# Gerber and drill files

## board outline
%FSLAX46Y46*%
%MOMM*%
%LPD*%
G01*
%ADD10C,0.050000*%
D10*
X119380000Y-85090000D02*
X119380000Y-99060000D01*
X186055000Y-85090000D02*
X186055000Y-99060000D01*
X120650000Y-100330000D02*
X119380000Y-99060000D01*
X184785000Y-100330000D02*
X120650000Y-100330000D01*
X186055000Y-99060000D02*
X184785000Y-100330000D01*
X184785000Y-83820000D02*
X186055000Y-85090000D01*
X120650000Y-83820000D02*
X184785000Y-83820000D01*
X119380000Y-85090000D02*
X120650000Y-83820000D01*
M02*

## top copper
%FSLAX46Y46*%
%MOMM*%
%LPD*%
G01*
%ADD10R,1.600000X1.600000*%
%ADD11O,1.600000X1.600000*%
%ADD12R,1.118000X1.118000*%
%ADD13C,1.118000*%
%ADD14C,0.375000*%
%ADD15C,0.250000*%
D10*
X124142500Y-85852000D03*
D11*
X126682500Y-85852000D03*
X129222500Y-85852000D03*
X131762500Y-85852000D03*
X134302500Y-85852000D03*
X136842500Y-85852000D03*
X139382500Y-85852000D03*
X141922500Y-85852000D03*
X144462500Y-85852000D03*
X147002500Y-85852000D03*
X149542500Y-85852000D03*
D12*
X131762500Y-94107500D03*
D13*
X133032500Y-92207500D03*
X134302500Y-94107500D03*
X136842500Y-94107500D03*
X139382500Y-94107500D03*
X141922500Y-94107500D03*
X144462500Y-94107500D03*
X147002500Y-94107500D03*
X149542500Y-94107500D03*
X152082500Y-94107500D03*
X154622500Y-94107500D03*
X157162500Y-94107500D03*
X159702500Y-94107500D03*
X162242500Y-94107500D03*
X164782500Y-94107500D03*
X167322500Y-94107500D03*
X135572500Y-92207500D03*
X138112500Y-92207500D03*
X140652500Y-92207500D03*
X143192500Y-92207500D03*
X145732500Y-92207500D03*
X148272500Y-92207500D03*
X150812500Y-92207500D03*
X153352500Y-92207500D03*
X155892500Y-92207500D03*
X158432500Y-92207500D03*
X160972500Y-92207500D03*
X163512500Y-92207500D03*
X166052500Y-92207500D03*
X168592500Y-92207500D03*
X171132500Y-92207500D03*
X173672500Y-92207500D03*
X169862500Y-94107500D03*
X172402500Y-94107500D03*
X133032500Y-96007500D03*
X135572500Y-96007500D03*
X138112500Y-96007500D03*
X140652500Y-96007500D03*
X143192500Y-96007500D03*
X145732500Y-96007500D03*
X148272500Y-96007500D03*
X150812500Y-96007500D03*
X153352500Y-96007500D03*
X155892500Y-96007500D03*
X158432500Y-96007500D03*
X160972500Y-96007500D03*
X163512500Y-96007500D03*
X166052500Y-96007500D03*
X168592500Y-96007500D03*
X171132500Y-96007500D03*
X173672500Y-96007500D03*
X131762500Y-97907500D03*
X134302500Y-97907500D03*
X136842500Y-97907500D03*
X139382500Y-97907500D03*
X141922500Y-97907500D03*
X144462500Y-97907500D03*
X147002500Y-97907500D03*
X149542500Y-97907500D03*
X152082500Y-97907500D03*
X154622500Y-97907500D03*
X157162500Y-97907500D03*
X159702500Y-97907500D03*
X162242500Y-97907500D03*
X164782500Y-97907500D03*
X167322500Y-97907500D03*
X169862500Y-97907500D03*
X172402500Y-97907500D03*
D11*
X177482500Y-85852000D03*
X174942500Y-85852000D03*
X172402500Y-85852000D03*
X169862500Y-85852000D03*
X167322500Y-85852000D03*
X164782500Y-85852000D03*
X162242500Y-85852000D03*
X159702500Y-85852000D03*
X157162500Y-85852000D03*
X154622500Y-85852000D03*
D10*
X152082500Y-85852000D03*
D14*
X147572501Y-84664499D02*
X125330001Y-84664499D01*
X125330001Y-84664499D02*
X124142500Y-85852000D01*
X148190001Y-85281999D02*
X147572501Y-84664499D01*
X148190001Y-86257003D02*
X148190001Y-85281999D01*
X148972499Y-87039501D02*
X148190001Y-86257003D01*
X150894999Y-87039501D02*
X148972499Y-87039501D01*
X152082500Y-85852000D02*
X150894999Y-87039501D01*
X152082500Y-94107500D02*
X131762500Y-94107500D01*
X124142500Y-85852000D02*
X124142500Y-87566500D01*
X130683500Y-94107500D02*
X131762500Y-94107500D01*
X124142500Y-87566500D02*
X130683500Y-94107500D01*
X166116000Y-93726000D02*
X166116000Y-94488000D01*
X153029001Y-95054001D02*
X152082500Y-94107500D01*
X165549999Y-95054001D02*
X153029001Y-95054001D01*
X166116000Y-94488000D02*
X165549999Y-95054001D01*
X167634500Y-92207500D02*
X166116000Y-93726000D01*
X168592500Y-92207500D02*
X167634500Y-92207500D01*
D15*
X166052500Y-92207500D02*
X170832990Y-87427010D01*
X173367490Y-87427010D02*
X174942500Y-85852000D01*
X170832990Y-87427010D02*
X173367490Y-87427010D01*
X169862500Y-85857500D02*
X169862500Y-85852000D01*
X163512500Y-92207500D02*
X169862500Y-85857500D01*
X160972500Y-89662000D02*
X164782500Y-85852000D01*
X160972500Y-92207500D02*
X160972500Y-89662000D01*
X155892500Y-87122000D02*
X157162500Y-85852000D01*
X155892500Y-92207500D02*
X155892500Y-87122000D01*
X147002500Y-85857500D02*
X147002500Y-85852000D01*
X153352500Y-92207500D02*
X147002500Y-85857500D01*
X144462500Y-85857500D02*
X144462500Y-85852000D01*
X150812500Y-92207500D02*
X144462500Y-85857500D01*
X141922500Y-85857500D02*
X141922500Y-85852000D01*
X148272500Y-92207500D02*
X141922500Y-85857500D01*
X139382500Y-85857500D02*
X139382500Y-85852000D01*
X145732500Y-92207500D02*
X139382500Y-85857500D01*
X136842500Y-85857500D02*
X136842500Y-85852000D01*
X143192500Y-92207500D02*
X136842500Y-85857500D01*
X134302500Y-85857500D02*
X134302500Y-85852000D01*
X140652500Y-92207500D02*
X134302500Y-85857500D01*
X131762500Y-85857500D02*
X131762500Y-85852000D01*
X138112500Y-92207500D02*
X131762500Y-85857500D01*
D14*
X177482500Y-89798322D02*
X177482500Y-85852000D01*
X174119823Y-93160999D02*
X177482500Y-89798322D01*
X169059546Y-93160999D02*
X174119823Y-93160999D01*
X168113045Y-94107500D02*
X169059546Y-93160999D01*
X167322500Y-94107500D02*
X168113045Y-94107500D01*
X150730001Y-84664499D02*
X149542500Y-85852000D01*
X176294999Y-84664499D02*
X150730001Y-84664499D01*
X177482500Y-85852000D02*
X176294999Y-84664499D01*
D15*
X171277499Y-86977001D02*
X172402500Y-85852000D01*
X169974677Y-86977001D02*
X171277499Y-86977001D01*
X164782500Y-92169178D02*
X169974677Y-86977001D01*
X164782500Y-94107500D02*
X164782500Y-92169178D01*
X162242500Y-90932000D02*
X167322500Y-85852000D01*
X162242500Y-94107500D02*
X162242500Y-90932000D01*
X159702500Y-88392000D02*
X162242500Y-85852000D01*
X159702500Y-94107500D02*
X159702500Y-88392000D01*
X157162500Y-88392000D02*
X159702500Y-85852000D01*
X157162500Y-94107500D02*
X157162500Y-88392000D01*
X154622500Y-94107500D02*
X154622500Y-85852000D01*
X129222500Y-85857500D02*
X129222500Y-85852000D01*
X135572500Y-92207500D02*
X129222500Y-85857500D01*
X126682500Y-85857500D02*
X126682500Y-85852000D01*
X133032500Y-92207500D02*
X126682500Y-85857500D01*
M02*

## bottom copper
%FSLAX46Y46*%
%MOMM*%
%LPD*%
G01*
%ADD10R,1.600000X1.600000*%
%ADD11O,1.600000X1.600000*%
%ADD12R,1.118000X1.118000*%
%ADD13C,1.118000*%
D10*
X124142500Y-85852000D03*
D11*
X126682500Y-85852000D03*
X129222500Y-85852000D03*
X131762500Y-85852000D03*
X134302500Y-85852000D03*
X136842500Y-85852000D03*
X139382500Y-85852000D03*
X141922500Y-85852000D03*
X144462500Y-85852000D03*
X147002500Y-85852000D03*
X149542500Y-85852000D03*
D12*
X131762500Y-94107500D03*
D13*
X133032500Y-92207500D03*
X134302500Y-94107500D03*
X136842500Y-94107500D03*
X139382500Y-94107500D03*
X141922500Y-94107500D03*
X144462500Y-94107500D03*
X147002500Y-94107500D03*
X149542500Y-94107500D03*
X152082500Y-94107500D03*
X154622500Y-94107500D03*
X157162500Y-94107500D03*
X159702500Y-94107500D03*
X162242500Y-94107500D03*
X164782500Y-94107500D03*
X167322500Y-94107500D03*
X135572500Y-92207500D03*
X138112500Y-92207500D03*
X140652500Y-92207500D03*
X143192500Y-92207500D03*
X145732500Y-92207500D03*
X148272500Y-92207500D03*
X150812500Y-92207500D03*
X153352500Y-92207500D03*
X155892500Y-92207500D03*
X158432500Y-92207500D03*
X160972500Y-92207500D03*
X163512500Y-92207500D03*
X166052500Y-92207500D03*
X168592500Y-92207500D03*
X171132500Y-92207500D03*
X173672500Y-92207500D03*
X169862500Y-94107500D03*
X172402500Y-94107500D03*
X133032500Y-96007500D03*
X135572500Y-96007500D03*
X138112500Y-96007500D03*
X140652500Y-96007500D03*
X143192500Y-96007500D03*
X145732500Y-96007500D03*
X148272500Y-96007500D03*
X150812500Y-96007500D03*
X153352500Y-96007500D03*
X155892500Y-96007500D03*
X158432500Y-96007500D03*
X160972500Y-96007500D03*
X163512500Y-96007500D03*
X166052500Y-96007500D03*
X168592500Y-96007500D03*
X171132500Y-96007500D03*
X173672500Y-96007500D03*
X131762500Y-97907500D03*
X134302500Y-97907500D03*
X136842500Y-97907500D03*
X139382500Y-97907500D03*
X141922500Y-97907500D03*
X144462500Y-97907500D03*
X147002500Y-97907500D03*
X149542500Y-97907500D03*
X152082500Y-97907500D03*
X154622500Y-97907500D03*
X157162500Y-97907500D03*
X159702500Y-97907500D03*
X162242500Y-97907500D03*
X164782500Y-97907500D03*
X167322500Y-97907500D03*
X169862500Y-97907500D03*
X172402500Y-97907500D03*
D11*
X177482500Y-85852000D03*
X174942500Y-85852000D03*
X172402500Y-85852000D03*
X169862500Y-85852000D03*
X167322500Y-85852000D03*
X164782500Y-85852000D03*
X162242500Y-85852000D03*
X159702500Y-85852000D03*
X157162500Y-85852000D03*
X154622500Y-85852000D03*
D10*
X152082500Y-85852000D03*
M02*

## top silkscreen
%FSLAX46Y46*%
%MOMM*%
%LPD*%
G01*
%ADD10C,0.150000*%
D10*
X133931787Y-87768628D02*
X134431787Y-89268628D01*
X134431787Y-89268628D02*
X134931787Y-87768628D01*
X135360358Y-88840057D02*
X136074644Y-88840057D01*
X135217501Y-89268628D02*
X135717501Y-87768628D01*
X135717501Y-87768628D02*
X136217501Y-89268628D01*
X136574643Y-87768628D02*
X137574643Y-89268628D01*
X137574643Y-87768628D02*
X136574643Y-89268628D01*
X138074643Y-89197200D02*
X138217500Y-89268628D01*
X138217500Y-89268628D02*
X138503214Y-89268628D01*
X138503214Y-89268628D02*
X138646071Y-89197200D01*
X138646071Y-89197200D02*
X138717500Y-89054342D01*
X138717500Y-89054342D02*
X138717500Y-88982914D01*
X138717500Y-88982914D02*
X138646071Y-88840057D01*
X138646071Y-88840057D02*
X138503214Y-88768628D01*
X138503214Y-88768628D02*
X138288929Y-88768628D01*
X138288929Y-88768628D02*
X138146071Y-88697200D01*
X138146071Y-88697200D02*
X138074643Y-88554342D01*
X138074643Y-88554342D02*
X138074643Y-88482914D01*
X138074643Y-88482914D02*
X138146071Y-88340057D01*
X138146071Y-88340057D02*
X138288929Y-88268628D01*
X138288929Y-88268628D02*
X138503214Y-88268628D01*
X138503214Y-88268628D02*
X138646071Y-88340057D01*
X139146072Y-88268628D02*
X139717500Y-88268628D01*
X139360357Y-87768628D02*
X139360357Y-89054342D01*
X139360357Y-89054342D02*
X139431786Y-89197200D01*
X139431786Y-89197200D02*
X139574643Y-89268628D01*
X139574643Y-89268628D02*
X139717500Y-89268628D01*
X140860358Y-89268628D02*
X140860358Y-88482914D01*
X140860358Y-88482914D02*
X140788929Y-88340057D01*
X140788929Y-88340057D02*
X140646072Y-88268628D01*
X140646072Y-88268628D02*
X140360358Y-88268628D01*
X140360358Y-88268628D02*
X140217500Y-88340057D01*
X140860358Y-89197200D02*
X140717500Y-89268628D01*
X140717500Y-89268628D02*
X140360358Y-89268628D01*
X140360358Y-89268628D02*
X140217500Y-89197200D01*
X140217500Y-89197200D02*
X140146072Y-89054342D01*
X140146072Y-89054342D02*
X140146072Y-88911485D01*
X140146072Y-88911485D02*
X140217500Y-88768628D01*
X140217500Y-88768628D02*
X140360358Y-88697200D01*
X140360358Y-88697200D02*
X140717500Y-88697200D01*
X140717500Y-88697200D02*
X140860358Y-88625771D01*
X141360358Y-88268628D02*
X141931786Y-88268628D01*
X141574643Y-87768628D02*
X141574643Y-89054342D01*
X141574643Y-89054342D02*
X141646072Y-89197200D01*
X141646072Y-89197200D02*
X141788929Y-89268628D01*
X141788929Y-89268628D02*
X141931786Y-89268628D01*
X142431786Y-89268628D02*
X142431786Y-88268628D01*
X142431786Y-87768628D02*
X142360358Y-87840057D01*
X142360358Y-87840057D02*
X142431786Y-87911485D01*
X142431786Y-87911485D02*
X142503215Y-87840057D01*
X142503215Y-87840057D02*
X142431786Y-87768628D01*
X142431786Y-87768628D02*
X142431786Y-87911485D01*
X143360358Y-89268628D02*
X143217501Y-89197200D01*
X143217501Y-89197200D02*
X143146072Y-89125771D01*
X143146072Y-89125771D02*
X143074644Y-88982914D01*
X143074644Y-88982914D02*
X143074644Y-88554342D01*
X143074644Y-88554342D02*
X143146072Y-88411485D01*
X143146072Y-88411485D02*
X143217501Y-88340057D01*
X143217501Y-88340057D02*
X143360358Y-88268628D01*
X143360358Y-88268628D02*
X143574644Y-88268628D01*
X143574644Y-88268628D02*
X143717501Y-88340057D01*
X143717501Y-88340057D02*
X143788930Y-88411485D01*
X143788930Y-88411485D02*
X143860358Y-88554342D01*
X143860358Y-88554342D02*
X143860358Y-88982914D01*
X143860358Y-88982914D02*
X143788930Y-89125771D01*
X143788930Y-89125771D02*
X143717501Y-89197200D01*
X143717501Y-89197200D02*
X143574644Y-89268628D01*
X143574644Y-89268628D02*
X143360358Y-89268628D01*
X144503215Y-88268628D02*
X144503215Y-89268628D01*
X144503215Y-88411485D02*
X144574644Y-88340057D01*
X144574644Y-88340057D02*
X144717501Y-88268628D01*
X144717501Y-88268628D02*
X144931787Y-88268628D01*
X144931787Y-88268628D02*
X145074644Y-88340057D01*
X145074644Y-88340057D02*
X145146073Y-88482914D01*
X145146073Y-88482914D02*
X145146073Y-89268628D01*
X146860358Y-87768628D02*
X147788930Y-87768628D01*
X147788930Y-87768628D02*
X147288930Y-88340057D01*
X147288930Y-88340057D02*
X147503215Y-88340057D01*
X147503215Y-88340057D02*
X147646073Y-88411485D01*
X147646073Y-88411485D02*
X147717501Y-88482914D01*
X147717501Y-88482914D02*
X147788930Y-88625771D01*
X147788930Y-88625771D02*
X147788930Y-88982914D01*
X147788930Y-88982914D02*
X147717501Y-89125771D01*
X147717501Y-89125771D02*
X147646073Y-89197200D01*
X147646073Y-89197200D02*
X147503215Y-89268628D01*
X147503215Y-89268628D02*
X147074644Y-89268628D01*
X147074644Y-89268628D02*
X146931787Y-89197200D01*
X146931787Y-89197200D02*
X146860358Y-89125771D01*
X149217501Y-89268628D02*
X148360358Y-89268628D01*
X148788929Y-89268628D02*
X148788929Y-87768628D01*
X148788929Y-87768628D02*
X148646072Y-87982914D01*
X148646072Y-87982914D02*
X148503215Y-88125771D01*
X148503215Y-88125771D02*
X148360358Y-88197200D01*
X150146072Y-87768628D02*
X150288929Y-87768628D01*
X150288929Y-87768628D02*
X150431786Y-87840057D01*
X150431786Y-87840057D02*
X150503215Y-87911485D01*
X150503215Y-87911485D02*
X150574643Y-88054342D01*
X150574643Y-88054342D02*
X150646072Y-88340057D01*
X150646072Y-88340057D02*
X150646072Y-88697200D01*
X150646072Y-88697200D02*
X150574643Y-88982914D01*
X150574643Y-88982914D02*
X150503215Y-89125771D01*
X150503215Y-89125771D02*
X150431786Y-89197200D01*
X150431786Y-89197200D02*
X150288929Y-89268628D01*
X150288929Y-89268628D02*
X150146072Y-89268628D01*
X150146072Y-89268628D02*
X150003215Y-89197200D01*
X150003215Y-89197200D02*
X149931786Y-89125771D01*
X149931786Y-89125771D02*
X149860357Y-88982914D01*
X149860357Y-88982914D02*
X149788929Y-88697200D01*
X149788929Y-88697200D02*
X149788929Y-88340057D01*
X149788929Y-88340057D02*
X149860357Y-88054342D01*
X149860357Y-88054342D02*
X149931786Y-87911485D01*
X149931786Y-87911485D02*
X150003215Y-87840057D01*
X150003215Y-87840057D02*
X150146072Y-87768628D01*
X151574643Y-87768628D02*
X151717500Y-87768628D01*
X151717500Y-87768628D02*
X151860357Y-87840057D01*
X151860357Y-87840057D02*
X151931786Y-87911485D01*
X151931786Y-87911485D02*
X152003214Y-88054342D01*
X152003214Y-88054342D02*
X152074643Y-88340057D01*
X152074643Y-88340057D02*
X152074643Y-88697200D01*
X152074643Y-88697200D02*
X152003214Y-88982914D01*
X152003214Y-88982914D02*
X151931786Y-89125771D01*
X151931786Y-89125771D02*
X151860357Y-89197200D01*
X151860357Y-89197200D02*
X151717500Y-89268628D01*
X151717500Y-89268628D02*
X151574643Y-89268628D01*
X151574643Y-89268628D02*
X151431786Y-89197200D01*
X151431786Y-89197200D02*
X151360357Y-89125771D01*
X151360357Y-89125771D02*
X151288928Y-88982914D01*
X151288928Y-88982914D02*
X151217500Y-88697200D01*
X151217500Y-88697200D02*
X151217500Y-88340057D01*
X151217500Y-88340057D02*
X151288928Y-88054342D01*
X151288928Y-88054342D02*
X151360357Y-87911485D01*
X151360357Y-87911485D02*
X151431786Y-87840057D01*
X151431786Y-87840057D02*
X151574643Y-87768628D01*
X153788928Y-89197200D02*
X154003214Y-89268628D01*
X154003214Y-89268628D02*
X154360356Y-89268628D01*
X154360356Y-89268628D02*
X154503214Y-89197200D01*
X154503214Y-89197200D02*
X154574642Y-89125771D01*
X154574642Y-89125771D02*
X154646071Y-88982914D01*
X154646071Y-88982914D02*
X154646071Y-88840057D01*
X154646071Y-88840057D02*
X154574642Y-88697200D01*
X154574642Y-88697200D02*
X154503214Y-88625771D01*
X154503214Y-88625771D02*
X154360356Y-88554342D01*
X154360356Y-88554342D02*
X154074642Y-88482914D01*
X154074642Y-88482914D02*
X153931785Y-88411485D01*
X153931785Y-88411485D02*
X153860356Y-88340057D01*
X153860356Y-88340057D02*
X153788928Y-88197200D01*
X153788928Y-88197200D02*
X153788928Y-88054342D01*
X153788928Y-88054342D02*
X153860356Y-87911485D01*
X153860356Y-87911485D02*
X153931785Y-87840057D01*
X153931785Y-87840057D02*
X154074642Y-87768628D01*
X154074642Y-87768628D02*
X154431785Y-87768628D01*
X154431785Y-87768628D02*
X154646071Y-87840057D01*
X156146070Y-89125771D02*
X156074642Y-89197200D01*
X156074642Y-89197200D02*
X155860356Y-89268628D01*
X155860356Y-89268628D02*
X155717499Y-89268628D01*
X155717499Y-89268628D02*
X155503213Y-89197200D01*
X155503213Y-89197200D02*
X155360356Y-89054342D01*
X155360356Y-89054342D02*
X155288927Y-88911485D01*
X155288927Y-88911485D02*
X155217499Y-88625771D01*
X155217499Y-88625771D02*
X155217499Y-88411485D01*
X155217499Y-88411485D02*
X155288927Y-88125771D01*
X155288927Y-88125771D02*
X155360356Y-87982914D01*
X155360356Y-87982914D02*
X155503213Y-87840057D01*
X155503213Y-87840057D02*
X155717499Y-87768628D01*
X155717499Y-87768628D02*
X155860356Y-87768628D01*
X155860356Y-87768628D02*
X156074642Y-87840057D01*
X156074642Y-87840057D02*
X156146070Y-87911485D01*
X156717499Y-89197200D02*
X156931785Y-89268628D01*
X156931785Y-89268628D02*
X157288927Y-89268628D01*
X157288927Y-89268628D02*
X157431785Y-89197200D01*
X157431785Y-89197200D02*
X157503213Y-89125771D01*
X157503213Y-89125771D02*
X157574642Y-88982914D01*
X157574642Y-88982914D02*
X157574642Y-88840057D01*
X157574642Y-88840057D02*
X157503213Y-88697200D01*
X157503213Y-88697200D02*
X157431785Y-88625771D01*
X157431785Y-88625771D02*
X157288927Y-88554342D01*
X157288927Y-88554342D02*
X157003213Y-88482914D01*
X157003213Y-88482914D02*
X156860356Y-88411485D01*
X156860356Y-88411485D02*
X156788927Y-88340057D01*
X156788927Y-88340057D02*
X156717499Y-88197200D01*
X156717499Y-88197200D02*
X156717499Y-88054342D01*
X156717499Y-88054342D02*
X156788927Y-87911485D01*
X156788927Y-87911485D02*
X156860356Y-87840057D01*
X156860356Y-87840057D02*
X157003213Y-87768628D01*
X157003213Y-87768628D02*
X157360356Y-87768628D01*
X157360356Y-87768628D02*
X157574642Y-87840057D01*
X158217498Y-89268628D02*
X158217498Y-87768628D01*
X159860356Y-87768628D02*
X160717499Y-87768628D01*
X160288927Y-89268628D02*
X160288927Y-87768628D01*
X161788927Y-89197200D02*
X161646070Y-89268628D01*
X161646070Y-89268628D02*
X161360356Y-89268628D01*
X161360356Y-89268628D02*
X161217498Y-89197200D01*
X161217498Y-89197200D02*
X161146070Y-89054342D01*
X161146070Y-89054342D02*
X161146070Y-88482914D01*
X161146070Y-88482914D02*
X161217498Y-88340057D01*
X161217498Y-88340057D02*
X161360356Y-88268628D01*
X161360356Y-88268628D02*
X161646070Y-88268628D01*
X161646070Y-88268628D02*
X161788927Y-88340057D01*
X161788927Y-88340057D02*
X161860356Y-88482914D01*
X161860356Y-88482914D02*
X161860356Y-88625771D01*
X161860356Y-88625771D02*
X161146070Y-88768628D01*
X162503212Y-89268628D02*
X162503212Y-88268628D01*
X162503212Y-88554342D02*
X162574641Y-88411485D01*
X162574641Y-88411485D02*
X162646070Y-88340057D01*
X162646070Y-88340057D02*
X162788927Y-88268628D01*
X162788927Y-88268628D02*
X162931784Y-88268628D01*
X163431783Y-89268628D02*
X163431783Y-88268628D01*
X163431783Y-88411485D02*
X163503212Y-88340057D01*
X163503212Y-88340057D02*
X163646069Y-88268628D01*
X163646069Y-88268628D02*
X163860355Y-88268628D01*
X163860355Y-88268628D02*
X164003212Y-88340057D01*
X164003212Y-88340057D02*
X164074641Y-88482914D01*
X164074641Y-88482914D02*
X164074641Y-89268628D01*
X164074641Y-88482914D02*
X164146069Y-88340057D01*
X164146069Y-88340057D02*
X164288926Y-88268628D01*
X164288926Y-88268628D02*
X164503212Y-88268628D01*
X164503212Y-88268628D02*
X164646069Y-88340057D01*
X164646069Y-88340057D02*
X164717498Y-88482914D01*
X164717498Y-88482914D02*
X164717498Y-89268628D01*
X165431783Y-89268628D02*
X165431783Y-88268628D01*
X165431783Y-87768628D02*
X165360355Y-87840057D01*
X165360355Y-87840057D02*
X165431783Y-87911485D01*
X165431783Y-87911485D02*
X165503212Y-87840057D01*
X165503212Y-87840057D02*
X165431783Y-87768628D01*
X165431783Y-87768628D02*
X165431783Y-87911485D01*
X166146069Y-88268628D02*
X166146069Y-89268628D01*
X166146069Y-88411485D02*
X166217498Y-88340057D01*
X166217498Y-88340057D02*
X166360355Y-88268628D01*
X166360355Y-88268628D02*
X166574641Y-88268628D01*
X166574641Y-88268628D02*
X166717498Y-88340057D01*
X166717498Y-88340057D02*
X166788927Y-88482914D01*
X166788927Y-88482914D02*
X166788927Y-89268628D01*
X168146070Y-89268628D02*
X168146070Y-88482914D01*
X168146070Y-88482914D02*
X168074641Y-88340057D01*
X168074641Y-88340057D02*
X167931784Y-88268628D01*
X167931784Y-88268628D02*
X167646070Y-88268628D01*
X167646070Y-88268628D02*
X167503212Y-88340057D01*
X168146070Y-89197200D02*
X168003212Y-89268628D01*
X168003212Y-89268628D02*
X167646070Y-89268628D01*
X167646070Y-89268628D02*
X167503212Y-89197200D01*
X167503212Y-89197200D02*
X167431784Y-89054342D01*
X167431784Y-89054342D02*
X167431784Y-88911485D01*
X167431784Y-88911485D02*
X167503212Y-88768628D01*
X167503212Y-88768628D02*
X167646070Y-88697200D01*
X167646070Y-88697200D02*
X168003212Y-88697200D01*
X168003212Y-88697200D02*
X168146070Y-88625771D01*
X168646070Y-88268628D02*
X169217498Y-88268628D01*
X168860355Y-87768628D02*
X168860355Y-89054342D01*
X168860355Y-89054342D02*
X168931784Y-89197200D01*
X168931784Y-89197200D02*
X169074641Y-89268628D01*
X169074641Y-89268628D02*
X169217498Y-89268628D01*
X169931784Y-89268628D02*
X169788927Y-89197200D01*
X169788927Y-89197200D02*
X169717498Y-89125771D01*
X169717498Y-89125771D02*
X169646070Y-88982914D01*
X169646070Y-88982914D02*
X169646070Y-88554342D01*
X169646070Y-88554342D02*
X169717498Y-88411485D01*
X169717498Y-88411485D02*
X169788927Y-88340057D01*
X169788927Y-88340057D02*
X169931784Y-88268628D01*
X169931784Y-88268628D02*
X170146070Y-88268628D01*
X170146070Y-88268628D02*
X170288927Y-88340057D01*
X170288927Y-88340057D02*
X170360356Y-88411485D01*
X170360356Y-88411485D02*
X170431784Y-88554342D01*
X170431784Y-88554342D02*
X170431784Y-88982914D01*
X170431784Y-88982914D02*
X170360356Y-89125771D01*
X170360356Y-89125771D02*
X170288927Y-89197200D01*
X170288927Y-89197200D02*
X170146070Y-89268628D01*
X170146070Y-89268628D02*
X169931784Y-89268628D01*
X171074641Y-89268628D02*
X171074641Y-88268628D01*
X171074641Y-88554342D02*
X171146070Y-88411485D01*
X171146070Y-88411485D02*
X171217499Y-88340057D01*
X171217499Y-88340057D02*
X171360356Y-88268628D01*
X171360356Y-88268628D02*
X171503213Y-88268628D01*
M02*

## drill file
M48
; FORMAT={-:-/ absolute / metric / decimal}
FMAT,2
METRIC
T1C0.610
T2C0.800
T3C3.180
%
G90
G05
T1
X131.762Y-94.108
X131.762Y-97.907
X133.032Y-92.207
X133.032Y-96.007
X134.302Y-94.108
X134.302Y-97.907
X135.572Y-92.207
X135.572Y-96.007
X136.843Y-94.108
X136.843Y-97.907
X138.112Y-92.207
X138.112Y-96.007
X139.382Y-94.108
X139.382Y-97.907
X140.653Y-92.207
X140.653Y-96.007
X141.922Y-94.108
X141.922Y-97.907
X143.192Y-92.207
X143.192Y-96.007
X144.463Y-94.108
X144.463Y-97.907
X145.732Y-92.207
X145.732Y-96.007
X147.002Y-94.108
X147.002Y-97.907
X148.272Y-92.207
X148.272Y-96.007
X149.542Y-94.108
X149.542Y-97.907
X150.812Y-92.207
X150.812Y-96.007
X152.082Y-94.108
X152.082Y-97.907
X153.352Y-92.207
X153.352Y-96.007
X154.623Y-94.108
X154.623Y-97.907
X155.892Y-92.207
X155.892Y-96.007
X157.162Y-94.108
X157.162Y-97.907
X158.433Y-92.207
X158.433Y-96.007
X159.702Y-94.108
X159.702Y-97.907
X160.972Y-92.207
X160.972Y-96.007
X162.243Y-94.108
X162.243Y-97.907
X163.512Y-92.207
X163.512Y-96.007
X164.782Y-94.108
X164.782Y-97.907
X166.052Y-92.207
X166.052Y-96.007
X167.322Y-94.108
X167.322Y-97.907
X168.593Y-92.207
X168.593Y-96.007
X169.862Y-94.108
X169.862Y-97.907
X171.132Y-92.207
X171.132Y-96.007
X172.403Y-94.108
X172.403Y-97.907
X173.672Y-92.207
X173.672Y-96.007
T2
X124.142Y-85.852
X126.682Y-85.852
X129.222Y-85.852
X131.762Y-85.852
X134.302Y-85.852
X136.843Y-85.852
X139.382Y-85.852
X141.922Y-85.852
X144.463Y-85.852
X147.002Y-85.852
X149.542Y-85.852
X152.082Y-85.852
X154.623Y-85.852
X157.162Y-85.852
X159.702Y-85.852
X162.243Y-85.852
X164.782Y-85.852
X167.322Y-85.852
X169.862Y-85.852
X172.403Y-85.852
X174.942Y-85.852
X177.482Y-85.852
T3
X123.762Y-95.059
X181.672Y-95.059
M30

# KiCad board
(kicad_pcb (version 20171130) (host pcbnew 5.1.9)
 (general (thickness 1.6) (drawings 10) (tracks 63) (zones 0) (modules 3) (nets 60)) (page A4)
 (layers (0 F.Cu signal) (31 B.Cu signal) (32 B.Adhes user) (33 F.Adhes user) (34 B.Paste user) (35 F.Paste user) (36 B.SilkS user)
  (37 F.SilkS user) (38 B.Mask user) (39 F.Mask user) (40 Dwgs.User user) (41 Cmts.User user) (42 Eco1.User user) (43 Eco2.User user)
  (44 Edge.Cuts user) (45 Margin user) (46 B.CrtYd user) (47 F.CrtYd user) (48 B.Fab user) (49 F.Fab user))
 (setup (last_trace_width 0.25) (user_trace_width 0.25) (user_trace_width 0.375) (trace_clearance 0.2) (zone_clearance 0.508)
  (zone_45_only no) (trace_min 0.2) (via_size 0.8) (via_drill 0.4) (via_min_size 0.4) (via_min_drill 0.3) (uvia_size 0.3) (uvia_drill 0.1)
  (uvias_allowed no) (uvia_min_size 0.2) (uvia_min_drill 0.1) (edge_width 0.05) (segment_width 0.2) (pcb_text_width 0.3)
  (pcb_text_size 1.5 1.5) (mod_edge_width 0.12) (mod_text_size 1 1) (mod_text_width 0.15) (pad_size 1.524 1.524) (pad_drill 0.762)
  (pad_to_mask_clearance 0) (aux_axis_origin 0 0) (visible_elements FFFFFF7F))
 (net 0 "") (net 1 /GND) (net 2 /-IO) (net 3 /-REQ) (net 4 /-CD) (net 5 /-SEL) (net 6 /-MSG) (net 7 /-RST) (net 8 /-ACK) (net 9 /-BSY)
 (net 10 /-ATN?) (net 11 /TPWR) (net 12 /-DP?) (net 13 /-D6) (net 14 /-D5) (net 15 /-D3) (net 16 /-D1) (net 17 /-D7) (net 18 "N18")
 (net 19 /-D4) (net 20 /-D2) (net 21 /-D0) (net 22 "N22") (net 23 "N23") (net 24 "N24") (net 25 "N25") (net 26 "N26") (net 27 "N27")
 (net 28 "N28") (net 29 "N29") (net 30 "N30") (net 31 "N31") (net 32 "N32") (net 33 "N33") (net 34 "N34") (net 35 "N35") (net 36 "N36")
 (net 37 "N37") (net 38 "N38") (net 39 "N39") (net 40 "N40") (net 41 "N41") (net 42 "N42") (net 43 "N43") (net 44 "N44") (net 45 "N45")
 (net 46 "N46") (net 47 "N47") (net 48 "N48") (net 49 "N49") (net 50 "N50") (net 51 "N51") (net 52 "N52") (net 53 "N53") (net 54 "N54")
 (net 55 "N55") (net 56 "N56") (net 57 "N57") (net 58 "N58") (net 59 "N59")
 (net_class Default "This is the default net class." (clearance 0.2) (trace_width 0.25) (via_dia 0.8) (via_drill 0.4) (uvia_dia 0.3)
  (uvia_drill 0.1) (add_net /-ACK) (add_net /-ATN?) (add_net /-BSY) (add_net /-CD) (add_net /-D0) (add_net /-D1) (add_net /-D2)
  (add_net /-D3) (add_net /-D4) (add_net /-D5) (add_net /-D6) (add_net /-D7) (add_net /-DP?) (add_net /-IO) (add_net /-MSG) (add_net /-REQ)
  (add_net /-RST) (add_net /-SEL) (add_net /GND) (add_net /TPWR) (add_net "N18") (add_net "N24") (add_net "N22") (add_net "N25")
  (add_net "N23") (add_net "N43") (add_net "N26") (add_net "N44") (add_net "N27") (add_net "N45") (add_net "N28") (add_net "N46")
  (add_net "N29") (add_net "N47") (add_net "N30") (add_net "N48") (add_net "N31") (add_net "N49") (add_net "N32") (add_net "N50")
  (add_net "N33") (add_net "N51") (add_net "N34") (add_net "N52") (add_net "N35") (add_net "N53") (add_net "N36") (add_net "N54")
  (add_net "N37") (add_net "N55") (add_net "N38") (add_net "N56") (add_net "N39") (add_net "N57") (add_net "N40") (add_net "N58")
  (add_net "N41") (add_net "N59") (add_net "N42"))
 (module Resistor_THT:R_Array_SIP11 (layer B.Cu) (at 124.1425 85.852)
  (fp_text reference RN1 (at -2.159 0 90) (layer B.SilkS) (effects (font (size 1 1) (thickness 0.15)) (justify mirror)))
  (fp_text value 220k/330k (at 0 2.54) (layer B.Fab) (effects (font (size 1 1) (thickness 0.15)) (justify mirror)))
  (pad 1 thru_hole rect (at 0 0) (size 1.6 1.6) (drill 0.8) (layers *.Cu *.Mask) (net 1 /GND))
  (pad 2 thru_hole oval (at 2.54 0) (size 1.6 1.6) (drill 0.8) (layers *.Cu *.Mask) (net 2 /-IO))
  (pad 3 thru_hole oval (at 5.08 0) (size 1.6 1.6) (drill 0.8) (layers *.Cu *.Mask) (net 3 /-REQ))
  (pad 4 thru_hole oval (at 7.62 0) (size 1.6 1.6) (drill 0.8) (layers *.Cu *.Mask) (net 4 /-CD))
  (pad 5 thru_hole oval (at 10.16 0) (size 1.6 1.6) (drill 0.8) (layers *.Cu *.Mask) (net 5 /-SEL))
  (pad 6 thru_hole oval (at 12.7 0) (size 1.6 1.6) (drill 0.8) (layers *.Cu *.Mask) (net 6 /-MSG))
  (pad 7 thru_hole oval (at 15.24 0) (size 1.6 1.6) (drill 0.8) (layers *.Cu *.Mask) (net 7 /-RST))
  (pad 8 thru_hole oval (at 17.78 0) (size 1.6 1.6) (drill 0.8) (layers *.Cu *.Mask) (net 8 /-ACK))
  (pad 9 thru_hole oval (at 20.32 0) (size 1.6 1.6) (drill 0.8) (layers *.Cu *.Mask) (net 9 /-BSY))
  (pad 10 thru_hole oval (at 22.86 0) (size 1.6 1.6) (drill 0.8) (layers *.Cu *.Mask) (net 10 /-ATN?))
  (pad 11 thru_hole oval (at 25.4 0) (size 1.6 1.6) (drill 0.8) (layers *.Cu *.Mask) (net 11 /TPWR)))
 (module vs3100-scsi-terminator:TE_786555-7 (layer B.Cu) (at 152.7175 95.0595 180)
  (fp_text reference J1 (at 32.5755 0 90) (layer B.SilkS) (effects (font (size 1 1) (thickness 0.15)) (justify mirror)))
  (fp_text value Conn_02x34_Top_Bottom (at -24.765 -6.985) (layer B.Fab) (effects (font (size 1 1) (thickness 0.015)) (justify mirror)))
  (pad None np_thru_hole circle (at -28.955 0 180) (size 3.18 3.18) (drill 3.18) (layers *.Cu *.Mask))
  (pad None np_thru_hole circle (at 28.955 0 180) (size 3.18 3.18) (drill 3.18) (layers *.Cu *.Mask))
  (pad 1 thru_hole rect (at 20.955 0.952 180) (size 1.118 1.118) (drill 0.61) (layers *.Cu *.Mask) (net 1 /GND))
  (pad 2 thru_hole circle (at 19.685 2.852 180) (size 1.118 1.118) (drill 0.61) (layers *.Cu *.Mask) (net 2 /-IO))
  (pad 3 thru_hole circle (at 18.415 0.952 180) (size 1.118 1.118) (drill 0.61) (layers *.Cu *.Mask) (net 1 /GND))
  (pad 5 thru_hole circle (at 15.875 0.952 180) (size 1.118 1.118) (drill 0.61) (layers *.Cu *.Mask) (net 1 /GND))
  (pad 7 thru_hole circle (at 13.335 0.952 180) (size 1.118 1.118) (drill 0.61) (layers *.Cu *.Mask) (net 1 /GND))
  (pad 9 thru_hole circle (at 10.795 0.952 180) (size 1.118 1.118) (drill 0.61) (layers *.Cu *.Mask) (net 1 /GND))
  (pad 11 thru_hole circle (at 8.255 0.952 180) (size 1.118 1.118) (drill 0.61) (layers *.Cu *.Mask) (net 1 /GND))
  (pad 13 thru_hole circle (at 5.715 0.952 180) (size 1.118 1.118) (drill 0.61) (layers *.Cu *.Mask) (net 1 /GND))
  (pad 15 thru_hole circle (at 3.175 0.952 180) (size 1.118 1.118) (drill 0.61) (layers *.Cu *.Mask) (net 1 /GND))
  (pad 17 thru_hole circle (at 0.635 0.952 180) (size 1.118 1.118) (drill 0.61) (layers *.Cu *.Mask) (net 1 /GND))
  (pad 19 thru_hole circle (at -1.905 0.952 180) (size 1.118 1.118) (drill 0.61) (layers *.Cu *.Mask) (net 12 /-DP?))
  (pad 21 thru_hole circle (at -4.445 0.952 180) (size 1.118 1.118) (drill 0.61) (layers *.Cu *.Mask) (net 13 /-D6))
  (pad 23 thru_hole circle (at -6.985 0.952 180) (size 1.118 1.118) (drill 0.61) (layers *.Cu *.Mask) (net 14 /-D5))
  (pad 25 thru_hole circle (at -9.525 0.952 180) (size 1.118 1.118) (drill 0.61) (layers *.Cu *.Mask) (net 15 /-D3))
  (pad 27 thru_hole circle (at -12.065 0.952 180) (size 1.118 1.118) (drill 0.61) (layers *.Cu *.Mask) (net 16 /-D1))
  (pad 29 thru_hole circle (at -14.605 0.952 180) (size 1.118 1.118) (drill 0.61) (layers *.Cu *.Mask) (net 11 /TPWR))
  (pad 4 thru_hole circle (at 17.145 2.852 180) (size 1.118 1.118) (drill 0.61) (layers *.Cu *.Mask) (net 3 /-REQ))
  (pad 6 thru_hole circle (at 14.605 2.852 180) (size 1.118 1.118) (drill 0.61) (layers *.Cu *.Mask) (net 4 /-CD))
  (pad 8 thru_hole circle (at 12.065 2.852 180) (size 1.118 1.118) (drill 0.61) (layers *.Cu *.Mask) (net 5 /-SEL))
  (pad 10 thru_hole circle (at 9.525 2.852 180) (size 1.118 1.118) (drill 0.61) (layers *.Cu *.Mask) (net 6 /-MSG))
  (pad 12 thru_hole circle (at 6.985 2.852 180) (size 1.118 1.118) (drill 0.61) (layers *.Cu *.Mask) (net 7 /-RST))
  (pad 14 thru_hole circle (at 4.445 2.852 180) (size 1.118 1.118) (drill 0.61) (layers *.Cu *.Mask) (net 8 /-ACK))
  (pad 16 thru_hole circle (at 1.905 2.852 180) (size 1.118 1.118) (drill 0.61) (layers *.Cu *.Mask) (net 9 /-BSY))
  (pad 18 thru_hole circle (at -0.635 2.852 180) (size 1.118 1.118) (drill 0.61) (layers *.Cu *.Mask) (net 10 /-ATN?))
  (pad 20 thru_hole circle (at -3.175 2.852 180) (size 1.118 1.118) (drill 0.61) (layers *.Cu *.Mask) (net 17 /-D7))
  (pad 22 thru_hole circle (at -5.715 2.852 180) (size 1.118 1.118) (drill 0.61) (layers *.Cu *.Mask) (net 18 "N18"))
  (pad 24 thru_hole circle (at -8.255 2.852 180) (size 1.118 1.118) (drill 0.61) (layers *.Cu *.Mask) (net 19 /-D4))
  (pad 26 thru_hole circle (at -10.795 2.852 180) (size 1.118 1.118) (drill 0.61) (layers *.Cu *.Mask) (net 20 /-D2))
  (pad 28 thru_hole circle (at -13.335 2.852 180) (size 1.118 1.118) (drill 0.61) (layers *.Cu *.Mask) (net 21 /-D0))
  (pad 30 thru_hole circle (at -15.875 2.852 180) (size 1.118 1.118) (drill 0.61) (layers *.Cu *.Mask) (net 1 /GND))
  (pad 32 thru_hole circle (at -18.415 2.852 180) (size 1.118 1.118) (drill 0.61) (layers *.Cu *.Mask) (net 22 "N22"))
  (pad 34 thru_hole circle (at -20.955 2.852 180) (size 1.118 1.118) (drill 0.61) (layers *.Cu *.Mask) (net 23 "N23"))
  (pad 31 thru_hole circle (at -17.145 0.952 180) (size 1.118 1.118) (drill 0.61) (layers *.Cu *.Mask) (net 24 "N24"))
  (pad 33 thru_hole circle (at -19.685 0.952 180) (size 1.118 1.118) (drill 0.61) (layers *.Cu *.Mask) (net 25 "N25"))
  (pad 36 thru_hole circle (at 19.685 -0.948 180) (size 1.118 1.118) (drill 0.61) (layers *.Cu *.Mask) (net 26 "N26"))
  (pad 38 thru_hole circle (at 17.145 -0.948 180) (size 1.118 1.118) (drill 0.61) (layers *.Cu *.Mask) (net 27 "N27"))
  (pad 40 thru_hole circle (at 14.605 -0.948 180) (size 1.118 1.118) (drill 0.61) (layers *.Cu *.Mask) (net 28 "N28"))
  (pad 42 thru_hole circle (at 12.065 -0.948 180) (size 1.118 1.118) (drill 0.61) (layers *.Cu *.Mask) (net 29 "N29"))
  (pad 44 thru_hole circle (at 9.525 -0.948 180) (size 1.118 1.118) (drill 0.61) (layers *.Cu *.Mask) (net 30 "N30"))
  (pad 46 thru_hole circle (at 6.985 -0.948 180) (size 1.118 1.118) (drill 0.61) (layers *.Cu *.Mask) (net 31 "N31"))
  (pad 48 thru_hole circle (at 4.445 -0.948 180) (size 1.118 1.118) (drill 0.61) (layers *.Cu *.Mask) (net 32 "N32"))
  (pad 50 thru_hole circle (at 1.905 -0.948 180) (size 1.118 1.118) (drill 0.61) (layers *.Cu *.Mask) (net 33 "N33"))
  (pad 52 thru_hole circle (at -0.635 -0.948 180) (size 1.118 1.118) (drill 0.61) (layers *.Cu *.Mask) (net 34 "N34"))
  (pad 54 thru_hole circle (at -3.175 -0.948 180) (size 1.118 1.118) (drill 0.61) (layers *.Cu *.Mask) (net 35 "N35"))
  (pad 56 thru_hole circle (at -5.715 -0.948 180) (size 1.118 1.118) (drill 0.61) (layers *.Cu *.Mask) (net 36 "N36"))
  (pad 58 thru_hole circle (at -8.255 -0.948 180) (size 1.118 1.118) (drill 0.61) (layers *.Cu *.Mask) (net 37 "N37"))
  (pad 60 thru_hole circle (at -10.795 -0.948 180) (size 1.118 1.118) (drill 0.61) (layers *.Cu *.Mask) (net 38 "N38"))
  (pad 62 thru_hole circle (at -13.335 -0.948 180) (size 1.118 1.118) (drill 0.61) (layers *.Cu *.Mask) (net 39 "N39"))
  (pad 64 thru_hole circle (at -15.875 -0.948 180) (size 1.118 1.118) (drill 0.61) (layers *.Cu *.Mask) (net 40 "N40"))
  (pad 66 thru_hole circle (at -18.415 -0.948 180) (size 1.118 1.118) (drill 0.61) (layers *.Cu *.Mask) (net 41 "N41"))
  (pad 68 thru_hole circle (at -20.955 -0.948 180) (size 1.118 1.118) (drill 0.61) (layers *.Cu *.Mask) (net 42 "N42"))
  (pad 35 thru_hole circle (at 20.955 -2.848 180) (size 1.118 1.118) (drill 0.61) (layers *.Cu *.Mask) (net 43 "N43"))
  (pad 37 thru_hole circle (at 18.415 -2.848 180) (size 1.118 1.118) (drill 0.61) (layers *.Cu *.Mask) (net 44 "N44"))
  (pad 39 thru_hole circle (at 15.875 -2.848 180) (size 1.118 1.118) (drill 0.61) (layers *.Cu *.Mask) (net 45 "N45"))
  (pad 41 thru_hole circle (at 13.335 -2.848 180) (size 1.118 1.118) (drill 0.61) (layers *.Cu *.Mask) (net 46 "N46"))
  (pad 43 thru_hole circle (at 10.795 -2.848 180) (size 1.118 1.118) (drill 0.61) (layers *.Cu *.Mask) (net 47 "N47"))
  (pad 45 thru_hole circle (at 8.255 -2.848 180) (size 1.118 1.118) (drill 0.61) (layers *.Cu *.Mask) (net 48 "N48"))
  (pad 47 thru_hole circle (at 5.715 -2.848 180) (size 1.118 1.118) (drill 0.61) (layers *.Cu *.Mask) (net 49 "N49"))
  (pad 49 thru_hole circle (at 3.175 -2.848 180) (size 1.118 1.118) (drill 0.61) (layers *.Cu *.Mask) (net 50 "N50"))
  (pad 51 thru_hole circle (at 0.635 -2.848 180) (size 1.118 1.118) (drill 0.61) (layers *.Cu *.Mask) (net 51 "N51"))
  (pad 53 thru_hole circle (at -1.905 -2.848 180) (size 1.118 1.118) (drill 0.61) (layers *.Cu *.Mask) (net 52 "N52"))
  (pad 55 thru_hole circle (at -4.445 -2.848 180) (size 1.118 1.118) (drill 0.61) (layers *.Cu *.Mask) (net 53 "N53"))
  (pad 57 thru_hole circle (at -6.985 -2.848 180) (size 1.118 1.118) (drill 0.61) (layers *.Cu *.Mask) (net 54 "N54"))
  (pad 59 thru_hole circle (at -9.525 -2.848 180) (size 1.118 1.118) (drill 0.61) (layers *.Cu *.Mask) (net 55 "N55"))
  (pad 61 thru_hole circle (at -12.065 -2.848 180) (size 1.118 1.118) (drill 0.61) (layers *.Cu *.Mask) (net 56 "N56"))
  (pad 63 thru_hole circle (at -14.605 -2.848 180) (size 1.118 1.118) (drill 0.61) (layers *.Cu *.Mask) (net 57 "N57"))
  (pad 65 thru_hole circle (at -17.145 -2.848 180) (size 1.118 1.118) (drill 0.61) (layers *.Cu *.Mask) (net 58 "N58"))
  (pad 67 thru_hole circle (at -19.685 -2.848 180) (size 1.118 1.118) (drill 0.61) (layers *.Cu *.Mask) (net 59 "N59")))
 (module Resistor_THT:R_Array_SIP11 (layer B.Cu) (at 152.0825 85.852)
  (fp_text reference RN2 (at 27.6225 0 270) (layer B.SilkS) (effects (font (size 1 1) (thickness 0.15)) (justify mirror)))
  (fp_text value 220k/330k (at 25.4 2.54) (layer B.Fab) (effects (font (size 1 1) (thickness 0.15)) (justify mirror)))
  (pad 11 thru_hole oval (at 25.4 0) (size 1.6 1.6) (drill 0.8) (layers *.Cu *.Mask) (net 11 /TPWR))
  (pad 10 thru_hole oval (at 22.86 0) (size 1.6 1.6) (drill 0.8) (layers *.Cu *.Mask) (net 21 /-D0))
  (pad 9 thru_hole oval (at 20.32 0) (size 1.6 1.6) (drill 0.8) (layers *.Cu *.Mask) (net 16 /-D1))
  (pad 8 thru_hole oval (at 17.78 0) (size 1.6 1.6) (drill 0.8) (layers *.Cu *.Mask) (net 20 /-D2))
  (pad 7 thru_hole oval (at 15.24 0) (size 1.6 1.6) (drill 0.8) (layers *.Cu *.Mask) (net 15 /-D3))
  (pad 6 thru_hole oval (at 12.7 0) (size 1.6 1.6) (drill 0.8) (layers *.Cu *.Mask) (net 19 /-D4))
  (pad 5 thru_hole oval (at 10.16 0) (size 1.6 1.6) (drill 0.8) (layers *.Cu *.Mask) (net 14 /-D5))
  (pad 4 thru_hole oval (at 7.62 0) (size 1.6 1.6) (drill 0.8) (layers *.Cu *.Mask) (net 13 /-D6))
  (pad 3 thru_hole oval (at 5.08 0) (size 1.6 1.6) (drill 0.8) (layers *.Cu *.Mask) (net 17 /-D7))
  (pad 2 thru_hole oval (at 2.54 0) (size 1.6 1.6) (drill 0.8) (layers *.Cu *.Mask) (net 12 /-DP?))
  (pad 1 thru_hole rect (at 0 0) (size 1.6 1.6) (drill 0.8) (layers *.Cu *.Mask) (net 1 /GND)))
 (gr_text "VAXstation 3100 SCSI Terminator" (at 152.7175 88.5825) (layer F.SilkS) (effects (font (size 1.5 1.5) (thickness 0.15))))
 (gr_line (start 119.38 85.09) (end 119.38 99.06) (layer Edge.Cuts) (width 0.05))
 (gr_line (start 186.055 85.09) (end 186.055 99.06) (layer Edge.Cuts) (width 0.05))
 (gr_line (start 120.65 100.33) (end 119.38 99.06) (layer Edge.Cuts) (width 0.05))
 (gr_line (start 184.785 100.33) (end 120.65 100.33) (layer Edge.Cuts) (width 0.05))
 (gr_line (start 186.055 99.06) (end 184.785 100.33) (layer Edge.Cuts) (width 0.05))
 (gr_line (start 184.785 83.82) (end 186.055 85.09) (layer Edge.Cuts) (width 0.05))
 (gr_line (start 120.65 83.82) (end 184.785 83.82) (layer Edge.Cuts) (width 0.05))
 (gr_line (start 119.38 85.09) (end 120.65 83.82) (layer Edge.Cuts) (width 0.05))
 (segment (start 147.572501 84.664499) (end 125.330001 84.664499) (width 0.375) (layer F.Cu) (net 1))
 (segment (start 125.330001 84.664499) (end 124.1425 85.852) (width 0.375) (layer F.Cu) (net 1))
 (segment (start 148.190001 85.281999) (end 147.572501 84.664499) (width 0.375) (layer F.Cu) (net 1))
 (segment (start 148.190001 86.257003) (end 148.190001 85.281999) (width 0.375) (layer F.Cu) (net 1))
 (segment (start 148.972499 87.039501) (end 148.190001 86.257003) (width 0.375) (layer F.Cu) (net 1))
 (segment (start 150.894999 87.039501) (end 148.972499 87.039501) (width 0.375) (layer F.Cu) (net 1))
 (segment (start 152.0825 85.852) (end 150.894999 87.039501) (width 0.375) (layer F.Cu) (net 1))
 (segment (start 152.0825 94.1075) (end 131.7625 94.1075) (width 0.375) (layer F.Cu) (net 1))
 (segment (start 124.1425 85.852) (end 124.1425 87.5665) (width 0.375) (layer F.Cu) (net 1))
 (segment (start 130.6835 94.1075) (end 131.7625 94.1075) (width 0.375) (layer F.Cu) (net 1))
 (segment (start 124.1425 87.5665) (end 130.6835 94.1075) (width 0.375) (layer F.Cu) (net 1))
 (segment (start 166.116 93.726) (end 166.116 94.488) (width 0.375) (layer F.Cu) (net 1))
 (segment (start 153.029001 95.054001) (end 152.0825 94.1075) (width 0.375) (layer F.Cu) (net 1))
 (segment (start 165.549999 95.054001) (end 153.029001 95.054001) (width 0.375) (layer F.Cu) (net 1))
 (segment (start 166.116 94.488) (end 165.549999 95.054001) (width 0.375) (layer F.Cu) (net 1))
 (segment (start 167.6345 92.2075) (end 166.116 93.726) (width 0.375) (layer F.Cu) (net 1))
 (segment (start 168.5925 92.2075) (end 167.6345 92.2075) (width 0.375) (layer F.Cu) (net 1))
 (segment (start 166.0525 92.2075) (end 170.83299 87.42701) (width 0.25) (layer F.Cu) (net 21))
 (segment (start 173.36749 87.42701) (end 174.9425 85.852) (width 0.25) (layer F.Cu) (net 21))
 (segment (start 170.83299 87.42701) (end 173.36749 87.42701) (width 0.25) (layer F.Cu) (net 21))
 (segment (start 169.8625 85.8575) (end 169.8625 85.852) (width 0.25) (layer F.Cu) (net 20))
 (segment (start 163.5125 92.2075) (end 169.8625 85.8575) (width 0.25) (layer F.Cu) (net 20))
 (segment (start 160.9725 89.662) (end 164.7825 85.852) (width 0.25) (layer F.Cu) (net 19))
 (segment (start 160.9725 92.2075) (end 160.9725 89.662) (width 0.25) (layer F.Cu) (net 19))
 (segment (start 155.8925 87.122) (end 157.1625 85.852) (width 0.25) (layer F.Cu) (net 17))
 (segment (start 155.8925 92.2075) (end 155.8925 87.122) (width 0.25) (layer F.Cu) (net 17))
 (segment (start 147.0025 85.8575) (end 147.0025 85.852) (width 0.25) (layer F.Cu) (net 10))
 (segment (start 153.3525 92.2075) (end 147.0025 85.8575) (width 0.25) (layer F.Cu) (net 10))
 (segment (start 144.4625 85.8575) (end 144.4625 85.852) (width 0.25) (layer F.Cu) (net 9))
 (segment (start 150.8125 92.2075) (end 144.4625 85.8575) (width 0.25) (layer F.Cu) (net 9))
 (segment (start 141.9225 85.8575) (end 141.9225 85.852) (width 0.25) (layer F.Cu) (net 8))
 (segment (start 148.2725 92.2075) (end 141.9225 85.8575) (width 0.25) (layer F.Cu) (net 8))
 (segment (start 139.3825 85.8575) (end 139.3825 85.852) (width 0.25) (layer F.Cu) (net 7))
 (segment (start 145.7325 92.2075) (end 139.3825 85.8575) (width 0.25) (layer F.Cu) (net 7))
 (segment (start 136.8425 85.8575) (end 136.8425 85.852) (width 0.25) (layer F.Cu) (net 6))
 (segment (start 143.1925 92.2075) (end 136.8425 85.8575) (width 0.25) (layer F.Cu) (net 6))
 (segment (start 134.3025 85.8575) (end 134.3025 85.852) (width 0.25) (layer F.Cu) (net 5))
 (segment (start 140.6525 92.2075) (end 134.3025 85.8575) (width 0.25) (layer F.Cu) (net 5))
 (segment (start 131.7625 85.8575) (end 131.7625 85.852) (width 0.25) (layer F.Cu) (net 4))
 (segment (start 138.1125 92.2075) (end 131.7625 85.8575) (width 0.25) (layer F.Cu) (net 4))
 (segment (start 177.4825 89.798322) (end 177.4825 85.852) (width 0.375) (layer F.Cu) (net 11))
 (segment (start 174.119823 93.160999) (end 177.4825 89.798322) (width 0.375) (layer F.Cu) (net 11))
 (segment (start 169.059546 93.160999) (end 174.119823 93.160999) (width 0.375) (layer F.Cu) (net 11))
 (segment (start 168.113045 94.1075) (end 169.059546 93.160999) (width 0.375) (layer F.Cu) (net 11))
 (segment (start 167.3225 94.1075) (end 168.113045 94.1075) (width 0.375) (layer F.Cu) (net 11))
 (segment (start 150.730001 84.664499) (end 149.5425 85.852) (width 0.375) (layer F.Cu) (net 11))
 (segment (start 176.294999 84.664499) (end 150.730001 84.664499) (width 0.375) (layer F.Cu) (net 11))
 (segment (start 177.4825 85.852) (end 176.294999 84.664499) (width 0.375) (layer F.Cu) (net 11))
 (segment (start 171.277499 86.977001) (end 172.4025 85.852) (width 0.25) (layer F.Cu) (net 16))
 (segment (start 169.974677 86.977001) (end 171.277499 86.977001) (width 0.25) (layer F.Cu) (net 16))
 (segment (start 164.7825 92.169178) (end 169.974677 86.977001) (width 0.25) (layer F.Cu) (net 16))
 (segment (start 164.7825 94.1075) (end 164.7825 92.169178) (width 0.25) (layer F.Cu) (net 16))
 (segment (start 162.2425 90.932) (end 167.3225 85.852) (width 0.25) (layer F.Cu) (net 15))
 (segment (start 162.2425 94.1075) (end 162.2425 90.932) (width 0.25) (layer F.Cu) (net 15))
 (segment (start 159.7025 88.392) (end 162.2425 85.852) (width 0.25) (layer F.Cu) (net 14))
 (segment (start 159.7025 94.1075) (end 159.7025 88.392) (width 0.25) (layer F.Cu) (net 14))
 (segment (start 157.1625 88.392) (end 159.7025 85.852) (width 0.25) (layer F.Cu) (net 13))
 (segment (start 157.1625 94.1075) (end 157.1625 88.392) (width 0.25) (layer F.Cu) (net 13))
 (segment (start 154.6225 94.1075) (end 154.6225 85.852) (width 0.25) (layer F.Cu) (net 12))
 (segment (start 129.2225 85.8575) (end 129.2225 85.852) (width 0.25) (layer F.Cu) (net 3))
 (segment (start 135.5725 92.2075) (end 129.2225 85.8575) (width 0.25) (layer F.Cu) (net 3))
 (segment (start 126.6825 85.8575) (end 126.6825 85.852) (width 0.25) (layer F.Cu) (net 2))
 (segment (start 133.0325 92.2075) (end 126.6825 85.8575) (width 0.25) (layer F.Cu) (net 2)))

